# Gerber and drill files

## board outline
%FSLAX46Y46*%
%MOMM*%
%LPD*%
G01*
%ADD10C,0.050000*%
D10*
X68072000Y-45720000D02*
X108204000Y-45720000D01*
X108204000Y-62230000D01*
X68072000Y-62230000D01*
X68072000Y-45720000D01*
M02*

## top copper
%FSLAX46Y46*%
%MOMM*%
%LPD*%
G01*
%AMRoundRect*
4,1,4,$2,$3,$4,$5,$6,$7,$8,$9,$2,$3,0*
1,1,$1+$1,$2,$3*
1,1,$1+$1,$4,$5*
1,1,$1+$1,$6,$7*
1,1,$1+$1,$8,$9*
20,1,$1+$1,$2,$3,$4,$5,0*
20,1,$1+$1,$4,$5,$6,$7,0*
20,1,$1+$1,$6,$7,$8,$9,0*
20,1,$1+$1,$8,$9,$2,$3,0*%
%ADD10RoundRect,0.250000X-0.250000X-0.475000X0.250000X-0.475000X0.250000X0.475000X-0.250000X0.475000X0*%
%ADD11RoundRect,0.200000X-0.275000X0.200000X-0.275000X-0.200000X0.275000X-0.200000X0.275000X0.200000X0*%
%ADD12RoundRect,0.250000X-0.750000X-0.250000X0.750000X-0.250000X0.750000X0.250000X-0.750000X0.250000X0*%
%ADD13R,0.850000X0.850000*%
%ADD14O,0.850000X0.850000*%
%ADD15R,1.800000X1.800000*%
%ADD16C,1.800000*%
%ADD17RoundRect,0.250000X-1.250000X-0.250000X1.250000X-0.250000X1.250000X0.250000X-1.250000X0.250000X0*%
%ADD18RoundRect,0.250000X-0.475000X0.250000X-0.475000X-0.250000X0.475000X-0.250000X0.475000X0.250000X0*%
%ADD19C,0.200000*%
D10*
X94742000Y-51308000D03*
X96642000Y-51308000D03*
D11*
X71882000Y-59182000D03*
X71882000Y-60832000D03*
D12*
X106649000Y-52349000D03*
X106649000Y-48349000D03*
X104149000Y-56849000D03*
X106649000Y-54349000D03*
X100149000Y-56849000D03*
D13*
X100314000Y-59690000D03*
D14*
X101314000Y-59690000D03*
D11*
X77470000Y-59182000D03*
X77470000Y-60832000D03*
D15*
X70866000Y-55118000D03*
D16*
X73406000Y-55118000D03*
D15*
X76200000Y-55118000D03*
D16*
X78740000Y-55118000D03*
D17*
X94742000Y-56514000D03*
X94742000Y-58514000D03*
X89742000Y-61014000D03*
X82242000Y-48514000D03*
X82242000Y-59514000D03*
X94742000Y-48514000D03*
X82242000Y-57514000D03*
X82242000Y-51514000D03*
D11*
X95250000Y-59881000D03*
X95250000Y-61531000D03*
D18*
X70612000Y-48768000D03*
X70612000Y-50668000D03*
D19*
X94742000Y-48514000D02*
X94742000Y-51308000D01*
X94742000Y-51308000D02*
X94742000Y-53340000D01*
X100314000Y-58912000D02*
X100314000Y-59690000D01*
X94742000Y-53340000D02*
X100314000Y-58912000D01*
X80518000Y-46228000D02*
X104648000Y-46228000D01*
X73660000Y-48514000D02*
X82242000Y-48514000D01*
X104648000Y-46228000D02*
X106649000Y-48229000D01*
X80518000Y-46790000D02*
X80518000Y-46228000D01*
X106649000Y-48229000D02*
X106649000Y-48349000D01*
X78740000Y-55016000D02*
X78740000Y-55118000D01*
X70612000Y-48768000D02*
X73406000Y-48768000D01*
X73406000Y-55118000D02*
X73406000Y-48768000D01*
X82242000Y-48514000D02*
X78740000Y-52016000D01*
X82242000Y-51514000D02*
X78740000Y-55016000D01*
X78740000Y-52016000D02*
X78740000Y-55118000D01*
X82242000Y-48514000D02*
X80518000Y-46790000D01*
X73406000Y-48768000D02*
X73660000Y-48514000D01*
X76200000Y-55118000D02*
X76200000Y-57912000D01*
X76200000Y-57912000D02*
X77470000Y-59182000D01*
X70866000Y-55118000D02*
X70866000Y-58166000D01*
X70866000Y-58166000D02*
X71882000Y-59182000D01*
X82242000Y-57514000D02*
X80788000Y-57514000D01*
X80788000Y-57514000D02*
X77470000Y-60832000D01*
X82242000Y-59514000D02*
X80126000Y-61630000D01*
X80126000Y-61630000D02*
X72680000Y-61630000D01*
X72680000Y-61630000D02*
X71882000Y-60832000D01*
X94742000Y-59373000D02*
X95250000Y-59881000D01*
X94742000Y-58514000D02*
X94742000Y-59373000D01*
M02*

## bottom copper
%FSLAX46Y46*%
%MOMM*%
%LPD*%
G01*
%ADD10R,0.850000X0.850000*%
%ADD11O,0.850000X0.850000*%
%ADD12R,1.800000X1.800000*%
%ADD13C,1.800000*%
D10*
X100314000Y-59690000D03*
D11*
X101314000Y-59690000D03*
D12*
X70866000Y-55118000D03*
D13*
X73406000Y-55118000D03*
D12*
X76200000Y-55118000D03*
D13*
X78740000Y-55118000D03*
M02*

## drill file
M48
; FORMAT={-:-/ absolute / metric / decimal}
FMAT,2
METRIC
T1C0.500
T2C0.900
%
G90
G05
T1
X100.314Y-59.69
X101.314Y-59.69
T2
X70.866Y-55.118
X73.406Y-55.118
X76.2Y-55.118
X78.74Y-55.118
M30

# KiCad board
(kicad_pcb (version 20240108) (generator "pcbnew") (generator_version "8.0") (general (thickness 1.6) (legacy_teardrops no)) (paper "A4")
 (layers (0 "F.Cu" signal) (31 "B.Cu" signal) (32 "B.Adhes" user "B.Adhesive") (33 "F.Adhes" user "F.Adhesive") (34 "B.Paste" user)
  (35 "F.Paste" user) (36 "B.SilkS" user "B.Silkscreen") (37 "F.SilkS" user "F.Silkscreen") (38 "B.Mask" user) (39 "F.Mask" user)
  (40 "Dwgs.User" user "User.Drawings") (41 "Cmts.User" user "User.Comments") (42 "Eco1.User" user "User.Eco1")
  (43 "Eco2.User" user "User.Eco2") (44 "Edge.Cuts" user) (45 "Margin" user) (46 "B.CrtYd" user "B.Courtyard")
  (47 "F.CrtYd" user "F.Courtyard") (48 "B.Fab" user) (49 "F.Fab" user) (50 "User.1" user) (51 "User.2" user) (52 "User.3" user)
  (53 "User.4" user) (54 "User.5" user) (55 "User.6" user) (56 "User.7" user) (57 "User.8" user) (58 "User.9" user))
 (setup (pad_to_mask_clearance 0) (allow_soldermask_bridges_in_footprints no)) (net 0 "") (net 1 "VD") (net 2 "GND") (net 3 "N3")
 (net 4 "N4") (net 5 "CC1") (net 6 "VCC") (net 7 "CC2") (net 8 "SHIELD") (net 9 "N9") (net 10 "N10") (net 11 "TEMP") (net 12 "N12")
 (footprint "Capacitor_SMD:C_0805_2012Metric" (layer "F.Cu") (at 95.692 51.308)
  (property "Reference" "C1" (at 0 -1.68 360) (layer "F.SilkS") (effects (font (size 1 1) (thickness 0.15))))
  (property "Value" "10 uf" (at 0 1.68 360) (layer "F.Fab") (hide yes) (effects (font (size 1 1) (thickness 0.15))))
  (pad "1" smd roundrect (at -0.95 0) (size 1 1.45) (layers "F.Cu" "F.Paste" "F.Mask") (roundrect_rratio 0.25) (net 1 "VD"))
  (pad "2" smd roundrect (at 0.95 0) (size 1 1.45) (layers "F.Cu" "F.Paste" "F.Mask") (roundrect_rratio 0.25) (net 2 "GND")))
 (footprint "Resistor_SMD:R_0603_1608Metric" (layer "F.Cu") (at 71.882 60.007 -90)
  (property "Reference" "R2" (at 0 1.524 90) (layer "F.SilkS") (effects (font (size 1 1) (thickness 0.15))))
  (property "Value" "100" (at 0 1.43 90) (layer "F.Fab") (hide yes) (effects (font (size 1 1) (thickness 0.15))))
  (pad "1" smd roundrect (at -0.825 0 270) (size 0.8 0.95) (layers "F.Cu" "F.Paste" "F.Mask") (roundrect_rratio 0.25) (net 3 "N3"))
  (pad "2" smd roundrect (at 0.825 0 270) (size 0.8 0.95) (layers "F.Cu" "F.Paste" "F.Mask") (roundrect_rratio 0.25) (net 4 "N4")))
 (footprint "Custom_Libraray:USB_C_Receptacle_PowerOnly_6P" (layer "F.Cu") (at 106.649 56.849)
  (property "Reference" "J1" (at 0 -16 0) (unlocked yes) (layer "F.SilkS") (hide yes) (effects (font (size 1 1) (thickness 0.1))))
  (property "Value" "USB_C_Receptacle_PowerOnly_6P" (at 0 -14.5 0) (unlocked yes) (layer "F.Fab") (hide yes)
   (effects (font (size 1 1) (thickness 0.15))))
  (pad "A5" smd roundrect (at 0 -4.5) (size 2 1) (layers "F.Cu" "F.Paste" "F.Mask") (roundrect_rratio 0.25) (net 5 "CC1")
   (thermal_bridge_angle 45))
  (pad "A9" smd roundrect (at 0 -8.5) (size 2 1) (layers "F.Cu" "F.Paste" "F.Mask") (roundrect_rratio 0.25) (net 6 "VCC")
   (thermal_bridge_angle 45))
  (pad "A12" smd roundrect (at -2.5 0) (size 2 1) (layers "F.Cu" "F.Paste" "F.Mask") (roundrect_rratio 0.25) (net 2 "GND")
   (thermal_bridge_angle 45))
  (pad "B5" smd roundrect (at 0 -2.5) (size 2 1) (layers "F.Cu" "F.Paste" "F.Mask") (roundrect_rratio 0.25) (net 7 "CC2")
   (thermal_bridge_angle 45))
  (pad "S1" smd roundrect (at -6.5 0) (size 2 1) (layers "F.Cu" "F.Paste" "F.Mask") (roundrect_rratio 0.25) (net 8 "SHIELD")
   (thermal_bridge_angle 45)))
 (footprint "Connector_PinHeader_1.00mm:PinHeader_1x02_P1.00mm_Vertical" (layer "F.Cu") (at 100.314 59.69 90)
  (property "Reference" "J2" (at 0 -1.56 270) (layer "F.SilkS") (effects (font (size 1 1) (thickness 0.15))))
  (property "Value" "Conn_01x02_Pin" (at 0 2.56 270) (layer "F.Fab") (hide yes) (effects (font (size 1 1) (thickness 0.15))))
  (pad "1" thru_hole rect (at 0 0 90) (size 0.85 0.85) (drill 0.5) (layers "*.Cu" "*.Mask") (remove_unused_layers no) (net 1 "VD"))
  (pad "2" thru_hole oval (at 0 1 90) (size 0.85 0.85) (drill 0.5) (layers "*.Cu" "*.Mask") (remove_unused_layers no) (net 2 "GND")))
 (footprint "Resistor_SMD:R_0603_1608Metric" (layer "F.Cu") (at 77.47 60.007 -90)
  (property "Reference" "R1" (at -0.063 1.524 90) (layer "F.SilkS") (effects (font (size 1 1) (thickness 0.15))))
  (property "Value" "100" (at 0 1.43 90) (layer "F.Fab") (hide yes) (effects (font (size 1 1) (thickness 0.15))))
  (pad "1" smd roundrect (at -0.825 0 270) (size 0.8 0.95) (layers "F.Cu" "F.Paste" "F.Mask") (roundrect_rratio 0.25) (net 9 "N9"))
  (pad "2" smd roundrect (at 0.825 0 270) (size 0.8 0.95) (layers "F.Cu" "F.Paste" "F.Mask") (roundrect_rratio 0.25) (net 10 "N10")))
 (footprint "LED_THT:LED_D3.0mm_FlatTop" (layer "F.Cu") (at 70.866 55.118)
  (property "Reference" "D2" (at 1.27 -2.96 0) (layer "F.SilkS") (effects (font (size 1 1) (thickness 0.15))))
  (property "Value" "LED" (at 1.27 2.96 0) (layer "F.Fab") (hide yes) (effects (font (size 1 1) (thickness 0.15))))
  (pad "1" thru_hole rect (at 0 0) (size 1.8 1.8) (drill 0.9) (layers "*.Cu" "*.Mask") (remove_unused_layers no) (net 3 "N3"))
  (pad "2" thru_hole circle (at 2.54 0) (size 1.8 1.8) (drill 0.9) (layers "*.Cu" "*.Mask") (remove_unused_layers no) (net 6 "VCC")))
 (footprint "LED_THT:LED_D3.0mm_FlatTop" (layer "F.Cu") (at 76.2 55.118)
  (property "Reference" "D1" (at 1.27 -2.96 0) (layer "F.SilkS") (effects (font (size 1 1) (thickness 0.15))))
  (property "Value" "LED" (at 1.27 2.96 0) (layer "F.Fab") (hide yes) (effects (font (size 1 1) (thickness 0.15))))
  (pad "1" thru_hole rect (at 0 0) (size 1.8 1.8) (drill 0.9) (layers "*.Cu" "*.Mask") (remove_unused_layers no) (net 9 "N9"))
  (pad "2" thru_hole circle (at 2.54 0) (size 1.8 1.8) (drill 0.9) (layers "*.Cu" "*.Mask") (remove_unused_layers no) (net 6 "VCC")))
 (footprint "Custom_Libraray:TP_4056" (layer "F.Cu") (at 94.742 56.514)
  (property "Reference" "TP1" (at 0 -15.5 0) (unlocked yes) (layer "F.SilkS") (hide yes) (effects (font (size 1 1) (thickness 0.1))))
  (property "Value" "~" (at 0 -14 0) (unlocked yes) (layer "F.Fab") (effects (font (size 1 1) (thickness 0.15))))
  (pad "1" smd roundrect (at 0 0) (size 3 1) (layers "F.Cu" "F.Paste" "F.Mask" "Dwgs.User") (roundrect_rratio 0.25) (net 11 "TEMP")
   (thermal_bridge_angle 45))
  (pad "2" smd roundrect (at 0 2) (size 3 1) (layers "F.Cu" "F.Paste" "F.Mask" "Dwgs.User") (roundrect_rratio 0.25) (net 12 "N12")
   (thermal_bridge_angle 45))
  (pad "3" smd roundrect (at -5 4.5) (size 3 1) (layers "F.Cu" "F.Paste" "F.Mask" "Dwgs.User") (roundrect_rratio 0.25) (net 2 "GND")
   (thermal_bridge_angle 45))
  (pad "4" smd roundrect (at -12.5 -8) (size 3 1) (layers "F.Cu" "F.Paste" "F.Mask" "Dwgs.User") (roundrect_rratio 0.25) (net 6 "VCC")
   (thermal_bridge_angle 45))
  (pad "5" smd roundrect (at -12.5 3) (size 3 1) (layers "F.Cu" "F.Paste" "F.Mask" "Dwgs.User") (roundrect_rratio 0.25) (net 4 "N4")
   (thermal_bridge_angle 45))
  (pad "5" smd roundrect (at 0 -8) (size 3 1) (layers "F.Cu" "F.Paste" "F.Mask" "Dwgs.User") (roundrect_rratio 0.25) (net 1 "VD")
   (thermal_bridge_angle 45))
  (pad "7" smd roundrect (at -12.5 1) (size 3 1) (layers "F.Cu" "F.Paste" "F.Mask" "Dwgs.User") (roundrect_rratio 0.25) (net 10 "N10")
   (thermal_bridge_angle 45))
  (pad "8" smd roundrect (at -12.5 -5) (size 3 1) (layers "F.Cu" "F.Paste" "F.Mask" "Dwgs.User") (roundrect_rratio 0.25) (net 6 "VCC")
   (thermal_bridge_angle 45)))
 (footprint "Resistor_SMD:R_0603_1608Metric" (layer "F.Cu") (at 95.25 60.706 -90)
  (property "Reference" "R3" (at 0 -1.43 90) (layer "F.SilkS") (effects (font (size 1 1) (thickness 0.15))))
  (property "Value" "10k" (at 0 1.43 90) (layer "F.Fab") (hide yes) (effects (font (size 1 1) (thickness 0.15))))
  (pad "1" smd roundrect (at -0.825 0 270) (size 0.8 0.95) (layers "F.Cu" "F.Paste" "F.Mask") (roundrect_rratio 0.25) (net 12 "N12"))
  (pad "2" smd roundrect (at 0.825 0 270) (size 0.8 0.95) (layers "F.Cu" "F.Paste" "F.Mask") (roundrect_rratio 0.25) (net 2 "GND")))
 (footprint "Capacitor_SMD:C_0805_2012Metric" (layer "F.Cu") (at 70.612 49.718 -90)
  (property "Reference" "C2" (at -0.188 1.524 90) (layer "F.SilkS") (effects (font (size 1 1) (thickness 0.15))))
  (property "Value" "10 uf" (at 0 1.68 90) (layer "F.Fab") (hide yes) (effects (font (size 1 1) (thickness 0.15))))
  (pad "1" smd roundrect (at -0.95 0 270) (size 1 1.45) (layers "F.Cu" "F.Paste" "F.Mask") (roundrect_rratio 0.25) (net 6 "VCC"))
  (pad "2" smd roundrect (at 0.95 0 270) (size 1 1.45) (layers "F.Cu" "F.Paste" "F.Mask") (roundrect_rratio 0.25) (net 2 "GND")))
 (gr_rect (start 68.072 45.72) (end 108.204 62.23) (stroke (width 0.05) (type default)) (fill none) (layer "Edge.Cuts"))
 (segment (start 94.742 48.514) (end 94.742 51.308) (width 0.2) (layer "F.Cu") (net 1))
 (segment (start 94.742 51.308) (end 94.742 53.34) (width 0.2) (layer "F.Cu") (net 1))
 (segment (start 100.314 58.912) (end 100.314 59.69) (width 0.2) (layer "F.Cu") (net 1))
 (segment (start 94.742 53.34) (end 100.314 58.912) (width 0.2) (layer "F.Cu") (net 1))
 (segment (start 80.518 46.228) (end 104.648 46.228) (width 0.2) (layer "F.Cu") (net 6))
 (segment (start 73.66 48.514) (end 82.242 48.514) (width 0.2) (layer "F.Cu") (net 6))
 (segment (start 104.648 46.228) (end 106.649 48.229) (width 0.2) (layer "F.Cu") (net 6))
 (segment (start 80.518 46.79) (end 80.518 46.228) (width 0.2) (layer "F.Cu") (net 6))
 (segment (start 106.649 48.229) (end 106.649 48.349) (width 0.2) (layer "F.Cu") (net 6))
 (segment (start 78.74 55.016) (end 78.74 55.118) (width 0.2) (layer "F.Cu") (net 6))
 (segment (start 70.612 48.768) (end 73.406 48.768) (width 0.2) (layer "F.Cu") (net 6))
 (segment (start 73.406 55.118) (end 73.406 48.768) (width 0.2) (layer "F.Cu") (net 6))
 (segment (start 82.242 48.514) (end 78.74 52.016) (width 0.2) (layer "F.Cu") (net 6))
 (segment (start 82.242 51.514) (end 78.74 55.016) (width 0.2) (layer "F.Cu") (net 6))
 (segment (start 78.74 52.016) (end 78.74 55.118) (width 0.2) (layer "F.Cu") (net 6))
 (segment (start 82.242 48.514) (end 80.518 46.79) (width 0.2) (layer "F.Cu") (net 6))
 (segment (start 73.406 48.768) (end 73.66 48.514) (width 0.2) (layer "F.Cu") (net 6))
 (segment (start 76.2 55.118) (end 76.2 57.912) (width 0.2) (layer "F.Cu") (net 9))
 (segment (start 76.2 57.912) (end 77.47 59.182) (width 0.2) (layer "F.Cu") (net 9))
 (segment (start 70.866 55.118) (end 70.866 58.166) (width 0.2) (layer "F.Cu") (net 3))
 (segment (start 70.866 58.166) (end 71.882 59.182) (width 0.2) (layer "F.Cu") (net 3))
 (segment (start 82.242 57.514) (end 80.788 57.514) (width 0.2) (layer "F.Cu") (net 10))
 (segment (start 80.788 57.514) (end 77.47 60.832) (width 0.2) (layer "F.Cu") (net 10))
 (segment (start 82.242 59.514) (end 80.126 61.63) (width 0.2) (layer "F.Cu") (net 4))
 (segment (start 80.126 61.63) (end 72.68 61.63) (width 0.2) (layer "F.Cu") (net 4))
 (segment (start 72.68 61.63) (end 71.882 60.832) (width 0.2) (layer "F.Cu") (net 4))
 (segment (start 94.742 59.373) (end 95.25 59.881) (width 0.2) (layer "F.Cu") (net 12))
 (segment (start 94.742 58.514) (end 94.742 59.373) (width 0.2) (layer "F.Cu") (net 12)))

